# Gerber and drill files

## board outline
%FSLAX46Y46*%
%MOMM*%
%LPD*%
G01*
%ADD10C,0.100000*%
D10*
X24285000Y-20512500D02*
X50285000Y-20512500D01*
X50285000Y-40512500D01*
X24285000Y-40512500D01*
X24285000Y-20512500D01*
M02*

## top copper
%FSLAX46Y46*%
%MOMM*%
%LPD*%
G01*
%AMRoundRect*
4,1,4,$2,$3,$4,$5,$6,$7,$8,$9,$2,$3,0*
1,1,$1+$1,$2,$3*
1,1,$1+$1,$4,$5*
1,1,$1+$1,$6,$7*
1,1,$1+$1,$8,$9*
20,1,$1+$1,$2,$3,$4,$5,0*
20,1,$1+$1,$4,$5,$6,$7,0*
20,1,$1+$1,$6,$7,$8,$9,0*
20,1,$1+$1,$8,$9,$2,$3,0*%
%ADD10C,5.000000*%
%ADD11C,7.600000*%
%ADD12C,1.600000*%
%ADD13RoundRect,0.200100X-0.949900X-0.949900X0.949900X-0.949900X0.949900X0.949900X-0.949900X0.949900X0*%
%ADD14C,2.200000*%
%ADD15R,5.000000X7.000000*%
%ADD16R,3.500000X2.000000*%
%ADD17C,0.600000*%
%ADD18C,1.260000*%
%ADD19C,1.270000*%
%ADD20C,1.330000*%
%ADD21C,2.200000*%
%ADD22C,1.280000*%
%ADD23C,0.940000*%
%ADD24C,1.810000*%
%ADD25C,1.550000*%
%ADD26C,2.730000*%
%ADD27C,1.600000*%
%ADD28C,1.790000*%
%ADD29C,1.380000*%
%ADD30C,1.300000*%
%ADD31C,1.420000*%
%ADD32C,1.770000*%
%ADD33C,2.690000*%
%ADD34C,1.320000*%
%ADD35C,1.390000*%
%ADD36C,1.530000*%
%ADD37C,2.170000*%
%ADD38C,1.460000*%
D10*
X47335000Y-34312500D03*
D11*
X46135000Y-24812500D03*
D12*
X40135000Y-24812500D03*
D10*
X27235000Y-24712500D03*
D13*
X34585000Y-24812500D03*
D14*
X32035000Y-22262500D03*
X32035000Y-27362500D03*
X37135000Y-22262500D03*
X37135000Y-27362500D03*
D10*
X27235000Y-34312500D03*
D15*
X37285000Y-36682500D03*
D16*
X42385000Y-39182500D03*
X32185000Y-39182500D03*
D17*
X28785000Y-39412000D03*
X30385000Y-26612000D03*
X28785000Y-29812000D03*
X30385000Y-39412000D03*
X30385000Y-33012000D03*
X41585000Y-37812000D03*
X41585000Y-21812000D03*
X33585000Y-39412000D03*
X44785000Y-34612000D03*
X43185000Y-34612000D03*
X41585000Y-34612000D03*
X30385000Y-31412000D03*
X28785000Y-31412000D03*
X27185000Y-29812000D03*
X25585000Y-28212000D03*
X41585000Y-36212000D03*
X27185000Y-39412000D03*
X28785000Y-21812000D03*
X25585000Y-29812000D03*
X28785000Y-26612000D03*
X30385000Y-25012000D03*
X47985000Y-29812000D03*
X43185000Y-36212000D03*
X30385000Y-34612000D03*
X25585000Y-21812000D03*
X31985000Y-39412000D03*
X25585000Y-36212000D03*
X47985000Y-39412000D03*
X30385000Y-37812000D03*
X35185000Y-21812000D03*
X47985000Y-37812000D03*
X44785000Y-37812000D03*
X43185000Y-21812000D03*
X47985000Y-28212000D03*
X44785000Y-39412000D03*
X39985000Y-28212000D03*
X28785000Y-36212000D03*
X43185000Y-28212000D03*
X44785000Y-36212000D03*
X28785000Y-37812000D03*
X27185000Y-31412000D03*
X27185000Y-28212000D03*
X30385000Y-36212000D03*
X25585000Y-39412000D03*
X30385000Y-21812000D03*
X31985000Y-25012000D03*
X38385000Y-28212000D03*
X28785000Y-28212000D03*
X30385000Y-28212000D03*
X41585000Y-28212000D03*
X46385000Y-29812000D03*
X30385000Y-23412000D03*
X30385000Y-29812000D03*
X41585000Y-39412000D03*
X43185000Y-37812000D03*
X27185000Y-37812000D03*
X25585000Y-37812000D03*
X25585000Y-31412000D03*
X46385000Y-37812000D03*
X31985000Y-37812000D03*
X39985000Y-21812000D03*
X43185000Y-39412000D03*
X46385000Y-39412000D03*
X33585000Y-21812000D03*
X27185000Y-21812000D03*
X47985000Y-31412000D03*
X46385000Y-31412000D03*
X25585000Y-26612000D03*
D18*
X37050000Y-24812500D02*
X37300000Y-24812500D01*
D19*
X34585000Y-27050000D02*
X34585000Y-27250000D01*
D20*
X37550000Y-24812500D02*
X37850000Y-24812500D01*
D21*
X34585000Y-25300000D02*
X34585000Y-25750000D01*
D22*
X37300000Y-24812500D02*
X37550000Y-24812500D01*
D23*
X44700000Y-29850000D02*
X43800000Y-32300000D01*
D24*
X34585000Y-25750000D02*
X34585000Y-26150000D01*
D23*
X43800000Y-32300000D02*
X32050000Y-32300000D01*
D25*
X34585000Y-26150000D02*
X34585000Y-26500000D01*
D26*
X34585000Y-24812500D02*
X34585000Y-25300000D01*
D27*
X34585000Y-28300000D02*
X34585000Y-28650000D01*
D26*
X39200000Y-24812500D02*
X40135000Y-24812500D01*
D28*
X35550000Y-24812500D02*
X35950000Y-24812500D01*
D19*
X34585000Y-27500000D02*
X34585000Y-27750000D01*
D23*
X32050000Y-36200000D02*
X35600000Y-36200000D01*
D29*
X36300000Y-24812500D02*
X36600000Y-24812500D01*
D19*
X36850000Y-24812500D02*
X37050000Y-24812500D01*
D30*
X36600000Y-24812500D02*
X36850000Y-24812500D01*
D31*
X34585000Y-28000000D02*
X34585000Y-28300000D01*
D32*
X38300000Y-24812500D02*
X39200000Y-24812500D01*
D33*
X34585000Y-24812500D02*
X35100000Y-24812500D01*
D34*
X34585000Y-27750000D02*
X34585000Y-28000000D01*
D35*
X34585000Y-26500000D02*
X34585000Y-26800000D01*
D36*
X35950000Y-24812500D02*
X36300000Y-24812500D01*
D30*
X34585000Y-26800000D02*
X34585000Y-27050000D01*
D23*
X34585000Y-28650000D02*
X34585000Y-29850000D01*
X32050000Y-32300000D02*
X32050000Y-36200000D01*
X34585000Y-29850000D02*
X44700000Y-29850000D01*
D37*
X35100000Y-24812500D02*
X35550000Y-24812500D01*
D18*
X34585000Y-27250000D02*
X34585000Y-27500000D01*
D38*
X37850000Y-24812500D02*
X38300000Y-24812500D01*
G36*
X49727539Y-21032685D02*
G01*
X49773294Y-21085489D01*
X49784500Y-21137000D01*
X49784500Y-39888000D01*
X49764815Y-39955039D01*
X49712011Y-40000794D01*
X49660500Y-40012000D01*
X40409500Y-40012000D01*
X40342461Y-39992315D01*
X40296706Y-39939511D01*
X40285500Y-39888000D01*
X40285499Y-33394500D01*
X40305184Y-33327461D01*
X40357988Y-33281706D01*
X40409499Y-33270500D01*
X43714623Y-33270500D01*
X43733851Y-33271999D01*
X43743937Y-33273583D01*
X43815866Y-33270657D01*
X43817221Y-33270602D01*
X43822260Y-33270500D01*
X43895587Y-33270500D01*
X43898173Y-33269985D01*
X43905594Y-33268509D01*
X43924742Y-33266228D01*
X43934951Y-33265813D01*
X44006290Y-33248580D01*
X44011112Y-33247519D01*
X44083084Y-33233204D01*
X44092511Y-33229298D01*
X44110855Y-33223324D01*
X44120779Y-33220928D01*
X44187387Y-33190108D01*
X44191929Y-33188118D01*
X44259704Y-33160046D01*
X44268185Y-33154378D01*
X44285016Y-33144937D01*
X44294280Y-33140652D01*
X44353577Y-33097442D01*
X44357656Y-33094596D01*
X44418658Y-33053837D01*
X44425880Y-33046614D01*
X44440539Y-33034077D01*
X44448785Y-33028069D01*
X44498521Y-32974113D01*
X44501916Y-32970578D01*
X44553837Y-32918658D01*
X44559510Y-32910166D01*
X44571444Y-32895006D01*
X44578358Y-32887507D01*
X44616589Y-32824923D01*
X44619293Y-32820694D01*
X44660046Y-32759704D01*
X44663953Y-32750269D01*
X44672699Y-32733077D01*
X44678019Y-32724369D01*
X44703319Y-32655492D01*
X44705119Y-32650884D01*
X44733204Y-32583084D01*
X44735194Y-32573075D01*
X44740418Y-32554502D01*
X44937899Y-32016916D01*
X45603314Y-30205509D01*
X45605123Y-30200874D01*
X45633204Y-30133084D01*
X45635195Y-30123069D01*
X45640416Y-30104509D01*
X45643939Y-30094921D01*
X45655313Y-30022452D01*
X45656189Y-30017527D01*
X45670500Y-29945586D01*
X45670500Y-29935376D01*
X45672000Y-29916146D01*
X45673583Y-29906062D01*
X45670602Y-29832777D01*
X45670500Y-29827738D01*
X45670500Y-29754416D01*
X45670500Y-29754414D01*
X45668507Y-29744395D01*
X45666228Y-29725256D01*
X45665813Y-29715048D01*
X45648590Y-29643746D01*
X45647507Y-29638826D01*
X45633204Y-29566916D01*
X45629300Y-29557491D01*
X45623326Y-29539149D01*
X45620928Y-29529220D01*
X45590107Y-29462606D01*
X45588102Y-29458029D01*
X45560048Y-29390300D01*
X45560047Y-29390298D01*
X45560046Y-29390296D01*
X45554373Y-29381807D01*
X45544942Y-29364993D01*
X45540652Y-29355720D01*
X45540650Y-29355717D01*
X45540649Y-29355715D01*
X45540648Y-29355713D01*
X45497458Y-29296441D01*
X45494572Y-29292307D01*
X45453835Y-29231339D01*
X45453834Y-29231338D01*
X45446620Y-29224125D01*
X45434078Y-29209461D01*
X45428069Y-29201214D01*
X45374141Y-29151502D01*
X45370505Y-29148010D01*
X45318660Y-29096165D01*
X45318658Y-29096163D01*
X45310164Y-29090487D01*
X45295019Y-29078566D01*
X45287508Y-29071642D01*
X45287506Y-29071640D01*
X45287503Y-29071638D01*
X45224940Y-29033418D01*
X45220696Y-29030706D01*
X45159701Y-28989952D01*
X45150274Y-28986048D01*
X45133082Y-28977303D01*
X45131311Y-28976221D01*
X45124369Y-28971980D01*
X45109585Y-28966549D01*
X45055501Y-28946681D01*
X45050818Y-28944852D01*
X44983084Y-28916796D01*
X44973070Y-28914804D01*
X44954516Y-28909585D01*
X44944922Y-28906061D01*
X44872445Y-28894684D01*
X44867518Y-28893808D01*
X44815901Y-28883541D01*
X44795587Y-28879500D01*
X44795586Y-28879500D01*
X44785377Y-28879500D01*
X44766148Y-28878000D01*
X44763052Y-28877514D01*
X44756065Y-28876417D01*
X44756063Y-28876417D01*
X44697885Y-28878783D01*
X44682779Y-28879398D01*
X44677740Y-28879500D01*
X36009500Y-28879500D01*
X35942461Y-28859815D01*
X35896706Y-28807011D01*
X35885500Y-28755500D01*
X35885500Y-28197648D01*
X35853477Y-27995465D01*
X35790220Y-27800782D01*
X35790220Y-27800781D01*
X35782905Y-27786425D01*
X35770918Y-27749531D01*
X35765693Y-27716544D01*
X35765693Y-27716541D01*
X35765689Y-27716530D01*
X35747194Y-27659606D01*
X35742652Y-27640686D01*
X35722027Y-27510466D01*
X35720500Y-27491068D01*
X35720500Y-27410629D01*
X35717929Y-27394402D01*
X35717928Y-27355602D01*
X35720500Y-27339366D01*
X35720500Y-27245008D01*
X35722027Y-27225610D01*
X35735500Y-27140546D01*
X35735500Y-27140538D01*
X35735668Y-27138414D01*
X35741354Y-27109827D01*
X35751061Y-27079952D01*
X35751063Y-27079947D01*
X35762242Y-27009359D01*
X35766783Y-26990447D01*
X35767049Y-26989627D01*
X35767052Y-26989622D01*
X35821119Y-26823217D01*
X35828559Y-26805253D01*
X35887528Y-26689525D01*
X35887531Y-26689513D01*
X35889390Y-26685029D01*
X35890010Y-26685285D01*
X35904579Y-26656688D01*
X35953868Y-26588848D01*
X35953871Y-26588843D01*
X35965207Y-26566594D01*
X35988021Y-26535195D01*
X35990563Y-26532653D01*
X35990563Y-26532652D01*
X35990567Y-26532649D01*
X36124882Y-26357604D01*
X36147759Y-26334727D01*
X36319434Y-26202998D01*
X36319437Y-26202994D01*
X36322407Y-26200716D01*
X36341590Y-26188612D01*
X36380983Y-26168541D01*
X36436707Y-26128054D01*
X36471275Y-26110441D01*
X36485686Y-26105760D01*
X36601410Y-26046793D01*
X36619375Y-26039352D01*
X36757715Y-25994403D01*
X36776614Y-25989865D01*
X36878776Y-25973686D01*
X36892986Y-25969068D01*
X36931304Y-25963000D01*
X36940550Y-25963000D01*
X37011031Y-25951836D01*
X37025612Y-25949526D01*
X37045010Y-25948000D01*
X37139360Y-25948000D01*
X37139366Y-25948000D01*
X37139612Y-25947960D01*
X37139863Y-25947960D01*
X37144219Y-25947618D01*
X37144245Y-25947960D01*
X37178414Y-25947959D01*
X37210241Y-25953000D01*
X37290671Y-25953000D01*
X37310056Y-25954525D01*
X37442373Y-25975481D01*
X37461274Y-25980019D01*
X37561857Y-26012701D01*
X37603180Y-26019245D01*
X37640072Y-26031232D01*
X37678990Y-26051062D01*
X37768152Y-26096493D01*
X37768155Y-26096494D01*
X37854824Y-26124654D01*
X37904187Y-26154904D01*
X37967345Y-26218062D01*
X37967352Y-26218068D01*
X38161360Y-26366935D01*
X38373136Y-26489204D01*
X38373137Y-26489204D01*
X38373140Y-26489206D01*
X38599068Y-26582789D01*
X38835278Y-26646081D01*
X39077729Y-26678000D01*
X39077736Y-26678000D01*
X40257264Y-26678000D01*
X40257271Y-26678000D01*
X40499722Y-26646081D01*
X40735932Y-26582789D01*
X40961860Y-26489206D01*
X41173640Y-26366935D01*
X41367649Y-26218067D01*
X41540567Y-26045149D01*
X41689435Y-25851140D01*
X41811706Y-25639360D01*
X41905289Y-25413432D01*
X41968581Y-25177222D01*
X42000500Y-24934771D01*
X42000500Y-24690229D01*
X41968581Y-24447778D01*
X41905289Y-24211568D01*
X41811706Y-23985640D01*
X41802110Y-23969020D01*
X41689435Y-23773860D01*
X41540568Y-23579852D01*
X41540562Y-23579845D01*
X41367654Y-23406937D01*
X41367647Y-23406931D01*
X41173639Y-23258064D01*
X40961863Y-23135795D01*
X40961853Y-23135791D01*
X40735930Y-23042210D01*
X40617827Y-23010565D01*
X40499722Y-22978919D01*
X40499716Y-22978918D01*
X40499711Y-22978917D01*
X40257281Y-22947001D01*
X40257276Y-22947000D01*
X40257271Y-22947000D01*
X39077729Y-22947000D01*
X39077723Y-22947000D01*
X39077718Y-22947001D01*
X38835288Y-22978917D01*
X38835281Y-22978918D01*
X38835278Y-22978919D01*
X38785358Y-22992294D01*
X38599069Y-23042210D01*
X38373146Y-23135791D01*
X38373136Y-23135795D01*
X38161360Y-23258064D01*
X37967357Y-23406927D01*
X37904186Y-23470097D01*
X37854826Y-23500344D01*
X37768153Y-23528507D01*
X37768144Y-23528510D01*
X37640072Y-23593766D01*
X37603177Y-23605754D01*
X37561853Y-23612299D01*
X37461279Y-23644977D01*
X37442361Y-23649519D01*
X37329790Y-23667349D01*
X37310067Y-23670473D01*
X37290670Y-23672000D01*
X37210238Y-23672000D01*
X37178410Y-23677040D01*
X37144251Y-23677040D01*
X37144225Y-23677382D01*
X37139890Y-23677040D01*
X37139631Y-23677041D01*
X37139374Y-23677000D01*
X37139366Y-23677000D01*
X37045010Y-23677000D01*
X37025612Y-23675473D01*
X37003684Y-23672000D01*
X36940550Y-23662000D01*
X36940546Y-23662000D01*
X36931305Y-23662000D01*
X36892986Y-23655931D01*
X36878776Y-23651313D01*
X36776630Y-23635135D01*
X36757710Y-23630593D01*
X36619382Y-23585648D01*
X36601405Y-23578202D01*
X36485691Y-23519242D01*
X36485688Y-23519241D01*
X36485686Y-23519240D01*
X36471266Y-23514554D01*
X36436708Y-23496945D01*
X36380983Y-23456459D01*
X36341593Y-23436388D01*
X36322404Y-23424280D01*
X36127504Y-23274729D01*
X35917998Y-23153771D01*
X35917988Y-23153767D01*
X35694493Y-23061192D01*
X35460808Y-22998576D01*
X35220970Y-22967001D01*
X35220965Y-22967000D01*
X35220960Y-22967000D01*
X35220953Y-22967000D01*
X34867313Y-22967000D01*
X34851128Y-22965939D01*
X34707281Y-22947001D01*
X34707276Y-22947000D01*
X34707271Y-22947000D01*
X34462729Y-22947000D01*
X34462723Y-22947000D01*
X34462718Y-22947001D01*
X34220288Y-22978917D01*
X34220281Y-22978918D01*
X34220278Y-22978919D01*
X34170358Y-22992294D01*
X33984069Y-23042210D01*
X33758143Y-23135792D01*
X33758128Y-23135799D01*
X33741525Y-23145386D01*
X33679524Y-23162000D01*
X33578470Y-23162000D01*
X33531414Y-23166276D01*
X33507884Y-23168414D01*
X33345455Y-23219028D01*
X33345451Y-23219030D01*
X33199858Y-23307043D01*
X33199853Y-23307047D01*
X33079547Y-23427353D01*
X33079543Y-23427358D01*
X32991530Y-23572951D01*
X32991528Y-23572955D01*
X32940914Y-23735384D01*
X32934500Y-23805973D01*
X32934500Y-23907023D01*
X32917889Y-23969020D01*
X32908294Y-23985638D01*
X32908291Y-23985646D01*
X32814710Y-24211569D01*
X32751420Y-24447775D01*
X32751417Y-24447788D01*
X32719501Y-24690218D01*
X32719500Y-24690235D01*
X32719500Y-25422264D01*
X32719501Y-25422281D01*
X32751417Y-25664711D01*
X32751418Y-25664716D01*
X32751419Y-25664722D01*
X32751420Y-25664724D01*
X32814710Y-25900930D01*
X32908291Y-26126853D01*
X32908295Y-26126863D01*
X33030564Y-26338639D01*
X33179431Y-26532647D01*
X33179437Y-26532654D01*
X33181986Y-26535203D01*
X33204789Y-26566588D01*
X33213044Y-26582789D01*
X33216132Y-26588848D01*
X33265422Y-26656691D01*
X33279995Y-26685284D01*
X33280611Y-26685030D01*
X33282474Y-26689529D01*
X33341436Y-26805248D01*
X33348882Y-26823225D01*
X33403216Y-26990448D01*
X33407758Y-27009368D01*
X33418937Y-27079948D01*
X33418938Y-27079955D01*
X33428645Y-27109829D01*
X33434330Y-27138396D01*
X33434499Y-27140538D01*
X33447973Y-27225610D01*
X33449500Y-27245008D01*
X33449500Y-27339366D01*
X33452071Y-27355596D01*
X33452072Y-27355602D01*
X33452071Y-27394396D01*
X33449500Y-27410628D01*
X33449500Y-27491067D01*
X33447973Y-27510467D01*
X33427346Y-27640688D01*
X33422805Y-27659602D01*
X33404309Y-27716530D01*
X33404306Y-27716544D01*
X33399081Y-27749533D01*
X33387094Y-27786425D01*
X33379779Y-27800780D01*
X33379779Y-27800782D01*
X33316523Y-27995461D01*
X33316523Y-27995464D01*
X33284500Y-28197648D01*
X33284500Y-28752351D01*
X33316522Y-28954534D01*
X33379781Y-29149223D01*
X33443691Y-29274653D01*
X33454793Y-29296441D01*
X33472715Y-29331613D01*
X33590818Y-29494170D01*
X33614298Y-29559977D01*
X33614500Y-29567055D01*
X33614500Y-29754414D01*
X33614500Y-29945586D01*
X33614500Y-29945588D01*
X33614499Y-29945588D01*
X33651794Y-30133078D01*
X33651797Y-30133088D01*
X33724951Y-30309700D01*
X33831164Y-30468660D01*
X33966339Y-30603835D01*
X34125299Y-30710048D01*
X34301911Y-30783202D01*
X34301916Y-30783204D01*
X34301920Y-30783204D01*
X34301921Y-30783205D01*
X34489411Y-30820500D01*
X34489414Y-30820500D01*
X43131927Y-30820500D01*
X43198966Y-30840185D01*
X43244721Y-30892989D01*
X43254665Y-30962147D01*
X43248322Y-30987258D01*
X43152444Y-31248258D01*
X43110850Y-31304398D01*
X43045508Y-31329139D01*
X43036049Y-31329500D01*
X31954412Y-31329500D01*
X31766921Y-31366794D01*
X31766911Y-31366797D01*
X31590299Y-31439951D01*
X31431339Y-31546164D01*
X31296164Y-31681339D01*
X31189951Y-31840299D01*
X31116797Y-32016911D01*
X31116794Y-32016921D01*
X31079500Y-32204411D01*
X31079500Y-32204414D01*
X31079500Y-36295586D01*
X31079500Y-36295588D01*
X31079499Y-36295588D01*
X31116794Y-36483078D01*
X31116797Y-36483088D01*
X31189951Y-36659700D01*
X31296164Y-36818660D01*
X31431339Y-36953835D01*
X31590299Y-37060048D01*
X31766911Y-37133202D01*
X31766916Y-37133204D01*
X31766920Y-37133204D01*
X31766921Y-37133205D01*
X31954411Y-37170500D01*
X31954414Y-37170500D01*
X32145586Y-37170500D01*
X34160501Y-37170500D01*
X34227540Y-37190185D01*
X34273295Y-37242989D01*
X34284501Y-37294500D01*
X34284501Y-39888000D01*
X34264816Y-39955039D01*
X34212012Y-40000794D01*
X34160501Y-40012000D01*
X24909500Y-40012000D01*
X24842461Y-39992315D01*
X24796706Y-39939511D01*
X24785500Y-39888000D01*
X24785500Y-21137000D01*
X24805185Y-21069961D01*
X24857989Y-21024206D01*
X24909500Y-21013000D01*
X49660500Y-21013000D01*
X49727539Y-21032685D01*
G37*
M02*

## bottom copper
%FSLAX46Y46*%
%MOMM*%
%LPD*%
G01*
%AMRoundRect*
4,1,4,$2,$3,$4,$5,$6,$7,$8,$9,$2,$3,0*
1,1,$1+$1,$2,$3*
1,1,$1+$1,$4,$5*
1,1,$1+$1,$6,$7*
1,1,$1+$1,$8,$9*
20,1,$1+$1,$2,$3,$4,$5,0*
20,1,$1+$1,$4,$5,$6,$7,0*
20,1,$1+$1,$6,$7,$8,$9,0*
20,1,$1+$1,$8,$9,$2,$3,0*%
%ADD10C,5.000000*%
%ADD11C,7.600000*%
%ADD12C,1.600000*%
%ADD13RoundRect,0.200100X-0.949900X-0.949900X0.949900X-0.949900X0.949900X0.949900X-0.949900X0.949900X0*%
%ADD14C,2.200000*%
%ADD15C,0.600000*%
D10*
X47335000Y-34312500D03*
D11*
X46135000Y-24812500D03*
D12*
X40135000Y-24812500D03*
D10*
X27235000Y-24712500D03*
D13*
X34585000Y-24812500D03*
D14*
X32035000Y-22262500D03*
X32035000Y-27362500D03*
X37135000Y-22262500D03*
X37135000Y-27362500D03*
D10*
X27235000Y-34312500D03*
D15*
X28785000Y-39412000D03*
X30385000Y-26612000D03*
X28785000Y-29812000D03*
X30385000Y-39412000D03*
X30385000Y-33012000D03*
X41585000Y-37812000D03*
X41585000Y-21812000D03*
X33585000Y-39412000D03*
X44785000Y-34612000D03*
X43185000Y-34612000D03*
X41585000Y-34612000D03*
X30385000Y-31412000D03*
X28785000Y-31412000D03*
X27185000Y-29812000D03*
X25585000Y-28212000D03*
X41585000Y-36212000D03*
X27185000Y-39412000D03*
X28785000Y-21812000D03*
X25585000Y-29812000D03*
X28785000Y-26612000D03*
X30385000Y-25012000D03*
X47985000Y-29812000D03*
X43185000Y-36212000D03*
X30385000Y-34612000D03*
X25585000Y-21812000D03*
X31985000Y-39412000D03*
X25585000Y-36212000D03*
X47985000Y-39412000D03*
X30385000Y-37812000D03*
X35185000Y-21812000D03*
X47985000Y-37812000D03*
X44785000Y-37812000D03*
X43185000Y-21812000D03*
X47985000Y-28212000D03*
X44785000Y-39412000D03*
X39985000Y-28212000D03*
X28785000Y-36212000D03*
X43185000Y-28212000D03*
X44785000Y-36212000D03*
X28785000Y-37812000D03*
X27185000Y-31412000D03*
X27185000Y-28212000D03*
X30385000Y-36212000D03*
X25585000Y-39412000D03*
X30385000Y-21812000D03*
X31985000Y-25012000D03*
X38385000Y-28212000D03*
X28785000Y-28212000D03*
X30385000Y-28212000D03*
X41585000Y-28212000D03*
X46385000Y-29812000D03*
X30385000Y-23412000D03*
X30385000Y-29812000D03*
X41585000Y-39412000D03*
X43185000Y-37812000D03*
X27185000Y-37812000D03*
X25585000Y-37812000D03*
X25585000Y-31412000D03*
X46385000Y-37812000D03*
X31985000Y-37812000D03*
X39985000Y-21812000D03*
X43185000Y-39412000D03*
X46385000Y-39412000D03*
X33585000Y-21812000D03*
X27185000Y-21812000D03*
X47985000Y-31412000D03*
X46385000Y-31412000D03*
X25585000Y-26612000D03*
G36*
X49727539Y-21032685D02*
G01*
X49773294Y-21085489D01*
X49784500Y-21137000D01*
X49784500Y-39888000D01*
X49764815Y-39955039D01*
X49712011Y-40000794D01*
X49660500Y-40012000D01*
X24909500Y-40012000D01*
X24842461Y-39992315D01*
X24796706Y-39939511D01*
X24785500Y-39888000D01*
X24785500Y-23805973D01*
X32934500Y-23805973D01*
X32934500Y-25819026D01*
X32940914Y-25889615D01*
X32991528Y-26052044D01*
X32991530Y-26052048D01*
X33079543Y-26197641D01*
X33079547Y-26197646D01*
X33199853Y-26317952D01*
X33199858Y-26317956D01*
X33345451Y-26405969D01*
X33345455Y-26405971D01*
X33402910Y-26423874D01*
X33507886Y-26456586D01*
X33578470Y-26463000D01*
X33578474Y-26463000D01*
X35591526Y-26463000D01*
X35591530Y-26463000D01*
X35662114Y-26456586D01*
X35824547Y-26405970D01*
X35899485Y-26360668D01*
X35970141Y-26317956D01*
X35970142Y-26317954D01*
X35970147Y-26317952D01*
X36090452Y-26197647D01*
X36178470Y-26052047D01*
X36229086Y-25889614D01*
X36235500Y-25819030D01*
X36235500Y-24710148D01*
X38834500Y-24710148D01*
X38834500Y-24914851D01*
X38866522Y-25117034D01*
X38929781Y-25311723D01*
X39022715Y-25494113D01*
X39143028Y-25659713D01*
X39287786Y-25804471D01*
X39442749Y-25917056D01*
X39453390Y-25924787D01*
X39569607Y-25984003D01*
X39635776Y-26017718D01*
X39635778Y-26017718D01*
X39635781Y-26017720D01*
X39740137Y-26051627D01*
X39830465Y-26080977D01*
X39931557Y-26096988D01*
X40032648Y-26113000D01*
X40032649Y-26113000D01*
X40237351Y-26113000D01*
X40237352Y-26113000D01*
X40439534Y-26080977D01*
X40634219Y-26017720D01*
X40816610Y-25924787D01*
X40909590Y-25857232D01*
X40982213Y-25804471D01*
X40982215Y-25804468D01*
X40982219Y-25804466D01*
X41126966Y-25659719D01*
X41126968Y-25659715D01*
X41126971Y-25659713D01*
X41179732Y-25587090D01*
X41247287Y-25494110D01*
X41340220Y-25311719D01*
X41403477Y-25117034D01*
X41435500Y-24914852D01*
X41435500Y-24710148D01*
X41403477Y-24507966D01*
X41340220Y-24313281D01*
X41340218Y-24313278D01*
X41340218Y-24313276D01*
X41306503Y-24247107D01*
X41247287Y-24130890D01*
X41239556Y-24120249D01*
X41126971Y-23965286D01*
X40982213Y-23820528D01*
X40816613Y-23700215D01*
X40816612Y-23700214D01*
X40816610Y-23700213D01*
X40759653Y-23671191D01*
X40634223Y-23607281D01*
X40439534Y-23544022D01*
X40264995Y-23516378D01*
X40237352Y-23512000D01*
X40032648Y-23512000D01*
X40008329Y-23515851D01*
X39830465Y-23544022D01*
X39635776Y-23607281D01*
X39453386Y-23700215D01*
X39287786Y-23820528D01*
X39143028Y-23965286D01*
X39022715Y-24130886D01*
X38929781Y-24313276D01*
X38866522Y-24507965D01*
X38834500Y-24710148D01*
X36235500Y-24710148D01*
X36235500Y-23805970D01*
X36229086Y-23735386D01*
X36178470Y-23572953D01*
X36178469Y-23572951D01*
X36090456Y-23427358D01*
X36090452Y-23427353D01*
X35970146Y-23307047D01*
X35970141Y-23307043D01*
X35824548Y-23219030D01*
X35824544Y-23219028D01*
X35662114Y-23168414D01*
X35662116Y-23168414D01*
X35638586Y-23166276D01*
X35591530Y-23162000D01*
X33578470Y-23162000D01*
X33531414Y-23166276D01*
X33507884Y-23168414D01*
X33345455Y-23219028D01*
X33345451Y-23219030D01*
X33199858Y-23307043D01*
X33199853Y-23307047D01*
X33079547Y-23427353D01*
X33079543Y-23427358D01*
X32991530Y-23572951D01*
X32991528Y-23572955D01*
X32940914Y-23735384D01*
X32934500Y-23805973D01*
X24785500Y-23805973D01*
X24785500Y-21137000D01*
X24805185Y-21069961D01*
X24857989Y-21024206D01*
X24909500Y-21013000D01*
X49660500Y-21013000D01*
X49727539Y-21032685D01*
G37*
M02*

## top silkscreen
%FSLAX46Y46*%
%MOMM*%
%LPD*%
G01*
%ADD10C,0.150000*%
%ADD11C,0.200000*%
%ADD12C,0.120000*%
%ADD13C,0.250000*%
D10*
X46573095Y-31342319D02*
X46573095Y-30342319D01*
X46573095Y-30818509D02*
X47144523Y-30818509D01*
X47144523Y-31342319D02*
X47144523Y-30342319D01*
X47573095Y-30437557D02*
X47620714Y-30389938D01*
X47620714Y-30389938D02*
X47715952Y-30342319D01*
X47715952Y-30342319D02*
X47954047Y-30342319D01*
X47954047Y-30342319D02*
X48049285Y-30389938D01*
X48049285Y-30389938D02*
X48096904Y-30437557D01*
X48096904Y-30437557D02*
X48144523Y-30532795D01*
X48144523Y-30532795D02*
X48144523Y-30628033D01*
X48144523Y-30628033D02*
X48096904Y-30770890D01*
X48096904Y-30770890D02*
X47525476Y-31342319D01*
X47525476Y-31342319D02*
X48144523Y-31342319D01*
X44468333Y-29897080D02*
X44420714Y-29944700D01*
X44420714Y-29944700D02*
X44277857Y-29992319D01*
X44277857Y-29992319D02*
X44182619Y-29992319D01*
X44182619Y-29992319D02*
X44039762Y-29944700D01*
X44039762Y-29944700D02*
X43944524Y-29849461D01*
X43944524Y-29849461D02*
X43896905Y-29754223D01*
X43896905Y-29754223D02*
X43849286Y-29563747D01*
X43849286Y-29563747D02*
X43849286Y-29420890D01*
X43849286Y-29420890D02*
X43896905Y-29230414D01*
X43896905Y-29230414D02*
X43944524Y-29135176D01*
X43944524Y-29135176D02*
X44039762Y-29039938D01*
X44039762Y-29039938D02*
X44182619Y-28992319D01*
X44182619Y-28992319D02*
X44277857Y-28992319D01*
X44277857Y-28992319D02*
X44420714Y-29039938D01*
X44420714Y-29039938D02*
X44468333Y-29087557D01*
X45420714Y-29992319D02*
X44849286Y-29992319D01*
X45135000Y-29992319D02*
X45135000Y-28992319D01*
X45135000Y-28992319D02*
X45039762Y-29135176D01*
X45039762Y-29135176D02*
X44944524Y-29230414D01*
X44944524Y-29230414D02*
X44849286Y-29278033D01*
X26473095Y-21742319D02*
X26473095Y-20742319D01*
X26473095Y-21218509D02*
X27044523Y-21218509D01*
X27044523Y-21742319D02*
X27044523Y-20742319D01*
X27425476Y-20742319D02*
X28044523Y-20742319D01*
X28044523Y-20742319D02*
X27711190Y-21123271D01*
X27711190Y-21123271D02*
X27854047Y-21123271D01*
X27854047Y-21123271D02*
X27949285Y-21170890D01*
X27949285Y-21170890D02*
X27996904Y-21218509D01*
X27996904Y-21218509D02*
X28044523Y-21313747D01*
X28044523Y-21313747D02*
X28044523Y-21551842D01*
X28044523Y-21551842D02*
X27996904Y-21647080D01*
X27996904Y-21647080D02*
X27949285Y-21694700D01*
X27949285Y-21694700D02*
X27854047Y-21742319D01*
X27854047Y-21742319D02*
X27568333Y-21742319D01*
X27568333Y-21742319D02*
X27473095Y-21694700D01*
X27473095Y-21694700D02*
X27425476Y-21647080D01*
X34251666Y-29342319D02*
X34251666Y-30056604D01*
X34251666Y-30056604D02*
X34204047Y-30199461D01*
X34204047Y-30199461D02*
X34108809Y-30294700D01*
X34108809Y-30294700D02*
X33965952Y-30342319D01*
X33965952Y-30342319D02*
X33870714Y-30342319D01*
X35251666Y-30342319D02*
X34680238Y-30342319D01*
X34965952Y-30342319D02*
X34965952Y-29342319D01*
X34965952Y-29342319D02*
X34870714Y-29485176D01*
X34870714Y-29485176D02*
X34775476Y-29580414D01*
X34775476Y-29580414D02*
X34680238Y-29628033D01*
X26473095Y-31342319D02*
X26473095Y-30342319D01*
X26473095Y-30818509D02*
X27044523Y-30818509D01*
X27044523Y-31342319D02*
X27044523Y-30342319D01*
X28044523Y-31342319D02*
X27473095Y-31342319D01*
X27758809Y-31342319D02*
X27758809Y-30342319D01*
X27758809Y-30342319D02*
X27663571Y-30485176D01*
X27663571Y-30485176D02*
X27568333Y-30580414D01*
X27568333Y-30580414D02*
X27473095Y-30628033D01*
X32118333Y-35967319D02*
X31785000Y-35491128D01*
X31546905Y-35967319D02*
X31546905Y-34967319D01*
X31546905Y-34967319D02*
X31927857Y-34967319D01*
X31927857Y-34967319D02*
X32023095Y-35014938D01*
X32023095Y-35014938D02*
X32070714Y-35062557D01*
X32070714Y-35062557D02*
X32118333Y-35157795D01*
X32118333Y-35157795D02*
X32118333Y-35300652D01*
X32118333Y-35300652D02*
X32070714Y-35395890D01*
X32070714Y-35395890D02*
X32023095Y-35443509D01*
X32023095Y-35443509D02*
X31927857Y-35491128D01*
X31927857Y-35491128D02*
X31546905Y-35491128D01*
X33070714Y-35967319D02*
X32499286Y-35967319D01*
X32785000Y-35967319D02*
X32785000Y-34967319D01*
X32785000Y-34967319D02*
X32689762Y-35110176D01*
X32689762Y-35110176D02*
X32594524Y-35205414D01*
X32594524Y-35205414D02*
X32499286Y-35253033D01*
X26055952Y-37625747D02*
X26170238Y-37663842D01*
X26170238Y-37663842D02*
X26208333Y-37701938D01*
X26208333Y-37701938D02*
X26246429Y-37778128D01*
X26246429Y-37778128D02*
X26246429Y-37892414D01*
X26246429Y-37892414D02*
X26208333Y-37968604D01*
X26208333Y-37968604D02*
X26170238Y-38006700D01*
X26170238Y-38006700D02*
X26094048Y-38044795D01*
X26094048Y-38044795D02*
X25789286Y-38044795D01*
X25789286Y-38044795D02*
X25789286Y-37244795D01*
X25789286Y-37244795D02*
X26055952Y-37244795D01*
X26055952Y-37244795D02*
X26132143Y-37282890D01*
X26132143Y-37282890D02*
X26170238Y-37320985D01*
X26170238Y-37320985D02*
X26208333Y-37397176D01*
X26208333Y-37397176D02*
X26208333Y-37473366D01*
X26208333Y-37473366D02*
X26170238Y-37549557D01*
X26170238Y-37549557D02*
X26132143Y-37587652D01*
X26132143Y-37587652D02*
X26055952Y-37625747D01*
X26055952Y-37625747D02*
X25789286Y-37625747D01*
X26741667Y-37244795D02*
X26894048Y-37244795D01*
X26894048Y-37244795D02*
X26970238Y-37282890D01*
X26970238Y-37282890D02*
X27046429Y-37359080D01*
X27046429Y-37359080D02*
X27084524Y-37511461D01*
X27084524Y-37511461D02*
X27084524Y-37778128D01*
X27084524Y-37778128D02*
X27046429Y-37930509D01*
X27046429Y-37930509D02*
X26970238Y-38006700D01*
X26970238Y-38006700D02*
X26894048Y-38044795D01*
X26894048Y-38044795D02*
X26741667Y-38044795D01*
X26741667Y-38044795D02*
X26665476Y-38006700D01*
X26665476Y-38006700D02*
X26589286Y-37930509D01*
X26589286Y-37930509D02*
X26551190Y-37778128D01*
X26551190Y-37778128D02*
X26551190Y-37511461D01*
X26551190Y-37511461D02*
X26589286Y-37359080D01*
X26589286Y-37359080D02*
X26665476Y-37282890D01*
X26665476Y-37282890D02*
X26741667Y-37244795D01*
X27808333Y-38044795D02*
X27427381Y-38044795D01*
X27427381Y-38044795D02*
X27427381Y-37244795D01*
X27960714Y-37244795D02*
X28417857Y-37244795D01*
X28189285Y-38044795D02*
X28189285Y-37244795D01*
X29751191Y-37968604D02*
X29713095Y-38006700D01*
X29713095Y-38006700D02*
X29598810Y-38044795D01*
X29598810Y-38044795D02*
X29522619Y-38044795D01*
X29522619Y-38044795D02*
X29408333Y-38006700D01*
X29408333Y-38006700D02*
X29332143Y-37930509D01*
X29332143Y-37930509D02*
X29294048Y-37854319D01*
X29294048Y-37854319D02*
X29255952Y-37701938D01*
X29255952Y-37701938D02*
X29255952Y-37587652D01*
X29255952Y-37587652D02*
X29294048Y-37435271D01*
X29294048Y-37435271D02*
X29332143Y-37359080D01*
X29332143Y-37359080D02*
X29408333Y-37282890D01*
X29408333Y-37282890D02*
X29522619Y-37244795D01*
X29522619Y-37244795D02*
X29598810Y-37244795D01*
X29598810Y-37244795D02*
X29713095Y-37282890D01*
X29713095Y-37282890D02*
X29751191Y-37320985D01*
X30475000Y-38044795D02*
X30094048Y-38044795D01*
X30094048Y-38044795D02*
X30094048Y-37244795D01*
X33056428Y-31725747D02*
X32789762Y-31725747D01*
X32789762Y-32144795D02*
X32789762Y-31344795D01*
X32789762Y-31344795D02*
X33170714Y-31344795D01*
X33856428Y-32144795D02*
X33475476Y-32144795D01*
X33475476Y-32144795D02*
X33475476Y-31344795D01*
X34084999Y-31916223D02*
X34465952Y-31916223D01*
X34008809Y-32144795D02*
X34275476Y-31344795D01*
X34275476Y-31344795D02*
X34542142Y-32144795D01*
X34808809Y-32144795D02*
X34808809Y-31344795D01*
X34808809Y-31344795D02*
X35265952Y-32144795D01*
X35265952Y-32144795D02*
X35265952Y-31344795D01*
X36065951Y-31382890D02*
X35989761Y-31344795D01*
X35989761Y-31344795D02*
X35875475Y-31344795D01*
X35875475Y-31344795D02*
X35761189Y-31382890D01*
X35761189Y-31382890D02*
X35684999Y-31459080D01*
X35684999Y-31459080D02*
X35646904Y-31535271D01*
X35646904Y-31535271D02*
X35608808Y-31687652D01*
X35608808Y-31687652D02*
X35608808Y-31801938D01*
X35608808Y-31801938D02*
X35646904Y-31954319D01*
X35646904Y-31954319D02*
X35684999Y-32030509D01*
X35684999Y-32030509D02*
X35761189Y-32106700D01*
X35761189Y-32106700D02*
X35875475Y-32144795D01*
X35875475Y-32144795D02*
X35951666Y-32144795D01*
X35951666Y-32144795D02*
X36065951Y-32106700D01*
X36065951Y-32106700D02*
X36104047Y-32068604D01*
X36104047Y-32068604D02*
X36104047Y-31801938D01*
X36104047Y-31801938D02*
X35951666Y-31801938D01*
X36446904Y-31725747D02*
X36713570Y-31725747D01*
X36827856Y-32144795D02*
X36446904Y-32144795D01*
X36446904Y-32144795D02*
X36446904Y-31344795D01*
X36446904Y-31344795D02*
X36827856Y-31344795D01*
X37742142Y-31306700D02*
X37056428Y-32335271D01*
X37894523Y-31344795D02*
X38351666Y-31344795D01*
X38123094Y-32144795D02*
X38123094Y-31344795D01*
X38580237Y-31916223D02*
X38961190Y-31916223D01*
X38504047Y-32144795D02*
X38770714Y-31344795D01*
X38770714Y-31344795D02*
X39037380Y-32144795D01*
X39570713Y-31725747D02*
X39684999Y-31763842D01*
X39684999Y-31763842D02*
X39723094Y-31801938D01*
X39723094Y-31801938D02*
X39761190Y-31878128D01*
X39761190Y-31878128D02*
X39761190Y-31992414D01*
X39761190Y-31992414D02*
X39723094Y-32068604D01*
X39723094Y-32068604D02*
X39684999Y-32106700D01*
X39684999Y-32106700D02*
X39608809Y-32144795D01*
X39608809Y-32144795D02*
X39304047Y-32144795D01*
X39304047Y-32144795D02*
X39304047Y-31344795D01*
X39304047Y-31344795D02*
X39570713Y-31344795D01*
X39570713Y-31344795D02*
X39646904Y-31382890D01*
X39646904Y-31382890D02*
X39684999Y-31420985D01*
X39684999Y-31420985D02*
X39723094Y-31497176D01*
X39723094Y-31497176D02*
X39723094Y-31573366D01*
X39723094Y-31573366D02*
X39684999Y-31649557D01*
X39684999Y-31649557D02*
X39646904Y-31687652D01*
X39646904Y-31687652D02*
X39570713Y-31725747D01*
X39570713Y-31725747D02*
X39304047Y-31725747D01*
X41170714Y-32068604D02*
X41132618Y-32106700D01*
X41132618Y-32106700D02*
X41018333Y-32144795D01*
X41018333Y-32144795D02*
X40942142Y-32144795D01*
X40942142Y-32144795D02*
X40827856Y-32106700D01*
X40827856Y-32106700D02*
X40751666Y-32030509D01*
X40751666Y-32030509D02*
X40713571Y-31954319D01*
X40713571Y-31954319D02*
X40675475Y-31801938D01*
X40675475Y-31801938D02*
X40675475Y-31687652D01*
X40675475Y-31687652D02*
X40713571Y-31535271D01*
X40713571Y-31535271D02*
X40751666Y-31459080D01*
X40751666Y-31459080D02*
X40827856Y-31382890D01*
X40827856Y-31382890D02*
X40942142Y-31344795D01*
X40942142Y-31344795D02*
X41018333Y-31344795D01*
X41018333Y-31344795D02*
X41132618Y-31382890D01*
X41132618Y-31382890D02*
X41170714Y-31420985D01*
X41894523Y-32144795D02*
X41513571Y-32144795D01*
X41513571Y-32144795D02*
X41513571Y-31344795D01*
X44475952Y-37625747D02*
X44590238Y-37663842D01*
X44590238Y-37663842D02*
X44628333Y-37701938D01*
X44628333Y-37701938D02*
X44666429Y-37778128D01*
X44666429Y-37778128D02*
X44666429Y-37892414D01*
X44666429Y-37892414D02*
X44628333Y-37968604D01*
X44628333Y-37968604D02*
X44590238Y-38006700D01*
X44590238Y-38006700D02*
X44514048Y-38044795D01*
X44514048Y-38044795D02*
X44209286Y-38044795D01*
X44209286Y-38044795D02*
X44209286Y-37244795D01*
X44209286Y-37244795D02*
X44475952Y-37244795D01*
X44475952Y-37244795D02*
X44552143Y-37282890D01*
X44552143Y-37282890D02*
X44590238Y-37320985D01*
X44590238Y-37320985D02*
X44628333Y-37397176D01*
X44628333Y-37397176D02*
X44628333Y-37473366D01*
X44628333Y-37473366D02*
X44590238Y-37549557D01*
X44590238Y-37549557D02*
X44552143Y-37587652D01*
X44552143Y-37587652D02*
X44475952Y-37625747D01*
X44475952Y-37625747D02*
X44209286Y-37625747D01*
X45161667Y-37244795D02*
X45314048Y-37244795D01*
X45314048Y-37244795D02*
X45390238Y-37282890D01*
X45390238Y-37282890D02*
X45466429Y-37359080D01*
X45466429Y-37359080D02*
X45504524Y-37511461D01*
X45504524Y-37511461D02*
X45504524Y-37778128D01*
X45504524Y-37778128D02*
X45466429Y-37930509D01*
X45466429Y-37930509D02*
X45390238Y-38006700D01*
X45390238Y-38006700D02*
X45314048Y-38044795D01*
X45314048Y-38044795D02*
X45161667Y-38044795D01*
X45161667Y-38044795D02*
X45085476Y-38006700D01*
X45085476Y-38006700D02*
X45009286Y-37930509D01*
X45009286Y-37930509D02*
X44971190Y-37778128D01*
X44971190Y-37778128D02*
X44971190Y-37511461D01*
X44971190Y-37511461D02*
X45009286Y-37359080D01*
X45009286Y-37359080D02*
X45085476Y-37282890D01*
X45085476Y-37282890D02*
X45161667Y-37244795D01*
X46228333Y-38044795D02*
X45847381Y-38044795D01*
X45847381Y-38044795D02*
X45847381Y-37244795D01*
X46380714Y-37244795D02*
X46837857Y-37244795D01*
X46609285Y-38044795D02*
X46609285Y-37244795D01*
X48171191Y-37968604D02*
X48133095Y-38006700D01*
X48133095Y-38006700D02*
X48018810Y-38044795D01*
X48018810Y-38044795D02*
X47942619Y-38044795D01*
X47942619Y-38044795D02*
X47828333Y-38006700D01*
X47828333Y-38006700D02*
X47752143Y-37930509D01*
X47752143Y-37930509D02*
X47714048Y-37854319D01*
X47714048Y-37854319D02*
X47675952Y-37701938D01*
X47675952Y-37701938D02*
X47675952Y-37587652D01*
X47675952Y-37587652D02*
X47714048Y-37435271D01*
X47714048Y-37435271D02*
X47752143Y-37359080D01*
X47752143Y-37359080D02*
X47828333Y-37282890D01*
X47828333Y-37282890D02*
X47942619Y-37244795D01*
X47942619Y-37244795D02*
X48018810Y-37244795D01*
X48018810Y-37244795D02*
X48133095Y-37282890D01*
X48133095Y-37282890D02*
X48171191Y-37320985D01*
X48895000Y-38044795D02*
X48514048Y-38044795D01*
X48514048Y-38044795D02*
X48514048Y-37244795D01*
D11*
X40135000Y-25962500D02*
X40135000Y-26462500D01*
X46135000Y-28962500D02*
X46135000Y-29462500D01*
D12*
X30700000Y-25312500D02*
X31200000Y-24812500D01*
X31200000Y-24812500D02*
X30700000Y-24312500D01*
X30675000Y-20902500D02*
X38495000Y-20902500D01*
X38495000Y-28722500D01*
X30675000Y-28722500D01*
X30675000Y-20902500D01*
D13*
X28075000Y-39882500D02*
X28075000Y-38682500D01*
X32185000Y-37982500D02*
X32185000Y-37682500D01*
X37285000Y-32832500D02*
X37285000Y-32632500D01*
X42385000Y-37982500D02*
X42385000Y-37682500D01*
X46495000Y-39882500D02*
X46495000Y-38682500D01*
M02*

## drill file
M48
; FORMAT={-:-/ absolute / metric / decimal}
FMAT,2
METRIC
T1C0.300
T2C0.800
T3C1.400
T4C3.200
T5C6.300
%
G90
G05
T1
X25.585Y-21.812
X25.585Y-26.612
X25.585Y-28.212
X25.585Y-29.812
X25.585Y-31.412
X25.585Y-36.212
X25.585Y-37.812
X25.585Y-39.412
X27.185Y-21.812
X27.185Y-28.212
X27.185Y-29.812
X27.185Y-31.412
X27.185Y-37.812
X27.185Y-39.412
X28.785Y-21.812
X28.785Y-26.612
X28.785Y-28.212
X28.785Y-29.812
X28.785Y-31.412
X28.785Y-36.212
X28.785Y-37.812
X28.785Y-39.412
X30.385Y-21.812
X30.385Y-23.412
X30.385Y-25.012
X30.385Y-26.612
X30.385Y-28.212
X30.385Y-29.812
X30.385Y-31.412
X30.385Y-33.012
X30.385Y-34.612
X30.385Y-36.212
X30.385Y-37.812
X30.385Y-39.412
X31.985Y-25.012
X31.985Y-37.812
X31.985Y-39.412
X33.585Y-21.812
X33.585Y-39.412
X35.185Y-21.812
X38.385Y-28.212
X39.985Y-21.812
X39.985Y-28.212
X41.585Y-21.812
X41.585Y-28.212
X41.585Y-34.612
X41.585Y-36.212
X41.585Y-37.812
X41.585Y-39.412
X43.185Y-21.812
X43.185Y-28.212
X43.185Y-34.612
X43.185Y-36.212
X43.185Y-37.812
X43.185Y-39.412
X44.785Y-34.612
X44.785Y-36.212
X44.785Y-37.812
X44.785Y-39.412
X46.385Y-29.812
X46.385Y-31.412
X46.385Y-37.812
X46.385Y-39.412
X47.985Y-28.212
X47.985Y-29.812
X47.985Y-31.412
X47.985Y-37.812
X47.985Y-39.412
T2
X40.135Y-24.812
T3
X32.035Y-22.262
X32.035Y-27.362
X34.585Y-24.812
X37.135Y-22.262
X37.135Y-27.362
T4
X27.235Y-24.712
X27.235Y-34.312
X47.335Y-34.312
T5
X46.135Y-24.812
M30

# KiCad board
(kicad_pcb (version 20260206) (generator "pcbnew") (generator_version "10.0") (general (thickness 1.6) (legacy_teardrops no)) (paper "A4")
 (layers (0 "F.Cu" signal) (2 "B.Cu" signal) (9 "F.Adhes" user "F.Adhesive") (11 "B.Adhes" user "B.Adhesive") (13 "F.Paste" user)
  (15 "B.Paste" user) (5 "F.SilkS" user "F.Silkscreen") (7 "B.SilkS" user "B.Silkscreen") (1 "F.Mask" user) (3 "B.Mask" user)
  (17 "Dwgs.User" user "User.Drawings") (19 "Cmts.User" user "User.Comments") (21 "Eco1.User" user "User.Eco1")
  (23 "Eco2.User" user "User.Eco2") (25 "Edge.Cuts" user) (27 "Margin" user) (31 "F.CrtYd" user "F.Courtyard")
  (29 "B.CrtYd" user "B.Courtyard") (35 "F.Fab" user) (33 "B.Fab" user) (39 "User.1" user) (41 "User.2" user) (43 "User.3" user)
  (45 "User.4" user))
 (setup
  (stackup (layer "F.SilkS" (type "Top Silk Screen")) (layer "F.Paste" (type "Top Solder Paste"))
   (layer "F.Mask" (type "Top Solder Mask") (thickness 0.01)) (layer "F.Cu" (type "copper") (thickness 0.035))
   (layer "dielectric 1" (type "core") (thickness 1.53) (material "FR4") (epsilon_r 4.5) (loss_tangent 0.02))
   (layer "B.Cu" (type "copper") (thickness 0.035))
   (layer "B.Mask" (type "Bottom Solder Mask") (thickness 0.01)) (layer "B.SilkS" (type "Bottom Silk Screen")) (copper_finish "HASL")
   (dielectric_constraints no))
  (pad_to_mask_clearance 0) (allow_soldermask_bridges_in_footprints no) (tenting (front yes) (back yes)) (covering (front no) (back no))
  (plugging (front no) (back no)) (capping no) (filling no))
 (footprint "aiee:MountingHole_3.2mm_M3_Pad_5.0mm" (layer "F.Cu") (at 47.335 34.3125)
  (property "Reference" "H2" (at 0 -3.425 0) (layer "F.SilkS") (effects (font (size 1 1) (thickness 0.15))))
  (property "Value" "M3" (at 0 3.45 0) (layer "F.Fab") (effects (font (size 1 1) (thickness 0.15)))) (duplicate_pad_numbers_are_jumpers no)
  (pad "1" thru_hole circle (at 0 0) (size 5 5) (drill 3.2) (layers "*.Cu" "*.Mask") (remove_unused_layers no) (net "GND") (zone_connect 2)))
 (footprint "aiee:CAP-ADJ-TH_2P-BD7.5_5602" (layer "F.Cu") (at 46.135 24.8125 180)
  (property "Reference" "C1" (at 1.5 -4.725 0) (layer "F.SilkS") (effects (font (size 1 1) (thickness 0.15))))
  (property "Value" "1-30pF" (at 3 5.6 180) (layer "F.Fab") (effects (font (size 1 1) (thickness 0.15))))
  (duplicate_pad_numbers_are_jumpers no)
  (fp_line (start 6 -1.15) (end 6 -1.65) (stroke (width 0.2) (type solid)) (layer "F.SilkS"))
  (fp_line (start 0 -4.15) (end 0 -4.65) (stroke (width 0.2) (type solid)) (layer "F.SilkS"))
  (pad "1" thru_hole circle (at 0 0 180) (size 7.6 7.6) (drill 6.3) (layers "*.Cu" "*.Mask") (remove_unused_layers no) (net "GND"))
  (pad "2" thru_hole circle (at 6 0 180) (size 1.6 1.6) (drill 0.8) (layers "*.Cu" "*.Mask") (remove_unused_layers no) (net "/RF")))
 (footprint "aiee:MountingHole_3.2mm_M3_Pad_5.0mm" (layer "F.Cu") (at 27.235 24.7125)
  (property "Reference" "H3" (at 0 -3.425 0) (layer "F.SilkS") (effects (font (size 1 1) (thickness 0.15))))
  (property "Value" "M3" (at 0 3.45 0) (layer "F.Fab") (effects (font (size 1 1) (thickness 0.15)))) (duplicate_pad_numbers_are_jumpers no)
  (pad "1" thru_hole circle (at 0 0) (size 5 5) (drill 3.2) (layers "*.Cu" "*.Mask") (remove_unused_layers no) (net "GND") (zone_connect 2)))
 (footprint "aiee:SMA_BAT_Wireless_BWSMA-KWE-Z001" (layer "F.Cu") (at 34.585 24.8125)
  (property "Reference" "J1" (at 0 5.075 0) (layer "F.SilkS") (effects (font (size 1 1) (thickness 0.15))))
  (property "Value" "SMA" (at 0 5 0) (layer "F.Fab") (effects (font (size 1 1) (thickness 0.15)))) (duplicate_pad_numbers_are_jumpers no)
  (fp_line (start -3.885 0.5) (end -3.385 0) (stroke (width 0.12) (type solid)) (layer "F.SilkS"))
  (fp_line (start -3.385 0) (end -3.885 -0.5) (stroke (width 0.12) (type solid)) (layer "F.SilkS"))
  (fp_rect (start -3.91 -3.91) (end 3.91 3.91) (stroke (width 0.12) (type default)) (fill no) (layer "F.SilkS"))
  (pad "1" thru_hole roundrect (at 0 0) (size 2.3 2.3) (drill 1.4) (layers "*.Cu" "*.Mask") (remove_unused_layers yes) (keep_end_layers yes)
   (zone_layer_connections) (roundrect_rratio 0.087) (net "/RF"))
  (pad "2" thru_hole circle (at -2.55 -2.55) (size 2.2 2.2) (drill 1.4) (layers "*.Cu" "*.Mask") (remove_unused_layers yes)
   (keep_end_layers yes) (zone_layer_connections) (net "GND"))
  (pad "2" thru_hole circle (at -2.55 2.55) (size 2.2 2.2) (drill 1.4) (layers "*.Cu" "*.Mask") (remove_unused_layers yes)
   (keep_end_layers yes) (zone_layer_connections) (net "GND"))
  (pad "2" thru_hole circle (at 2.55 -2.55) (size 2.2 2.2) (drill 1.4) (layers "*.Cu" "*.Mask") (remove_unused_layers yes)
   (keep_end_layers yes) (zone_layer_connections) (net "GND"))
  (pad "2" thru_hole circle (at 2.55 2.55) (size 2.2 2.2) (drill 1.4) (layers "*.Cu" "*.Mask") (remove_unused_layers yes)
   (keep_end_layers yes) (zone_layer_connections) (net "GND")))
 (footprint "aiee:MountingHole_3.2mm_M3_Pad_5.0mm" (layer "F.Cu") (at 27.235 34.3125)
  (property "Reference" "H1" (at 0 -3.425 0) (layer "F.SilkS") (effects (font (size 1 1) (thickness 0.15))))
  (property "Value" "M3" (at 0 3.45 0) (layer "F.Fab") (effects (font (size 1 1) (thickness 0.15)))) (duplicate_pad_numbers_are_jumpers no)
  (pad "1" thru_hole circle (at 0 0) (size 5 5) (drill 3.2) (layers "*.Cu" "*.Mask") (remove_unused_layers no) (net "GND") (zone_connect 2)))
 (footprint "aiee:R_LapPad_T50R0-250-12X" (layer "F.Cu") (at 37.285 40.1825 180)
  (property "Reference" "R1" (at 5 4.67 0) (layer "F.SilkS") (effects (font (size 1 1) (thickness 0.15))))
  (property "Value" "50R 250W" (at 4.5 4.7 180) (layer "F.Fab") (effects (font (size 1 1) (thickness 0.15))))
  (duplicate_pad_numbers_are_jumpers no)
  (fp_line (start 9.21 0.3) (end 9.21 1.5) (stroke (width 0.25) (type solid)) (layer "F.SilkS"))
  (fp_line (start 5.1 2.2) (end 5.1 2.5) (stroke (width 0.25) (type solid)) (layer "F.SilkS"))
  (fp_line (start 0 7.35) (end 0 7.55) (stroke (width 0.25) (type solid)) (layer "F.SilkS"))
  (fp_line (start -5.1 2.2) (end -5.1 2.5) (stroke (width 0.25) (type solid)) (layer "F.SilkS"))
  (fp_line (start -9.21 0.3) (end -9.21 1.5) (stroke (width 0.25) (type solid)) (layer "F.SilkS"))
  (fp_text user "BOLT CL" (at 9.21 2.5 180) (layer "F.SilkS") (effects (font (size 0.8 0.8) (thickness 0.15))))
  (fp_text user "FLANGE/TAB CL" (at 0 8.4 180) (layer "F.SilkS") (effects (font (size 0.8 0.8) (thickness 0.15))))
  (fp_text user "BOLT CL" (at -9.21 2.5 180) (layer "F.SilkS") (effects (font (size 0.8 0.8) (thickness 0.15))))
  (pad "1" smd rect (at 0 3.5 180) (size 5 7) (layers "F.Cu" "F.Mask" "F.Paste") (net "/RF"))
  (pad "2" smd rect (at -5.1 1 180) (size 3.5 2) (layers "F.Cu" "F.Mask" "F.Paste") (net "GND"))
  (pad "2" smd rect (at 5.1 1 180) (size 3.5 2) (layers "F.Cu" "F.Mask" "F.Paste") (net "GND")))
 (gr_rect (start 24.285 20.5125) (end 50.285 40.5125) (stroke (width 0.1) (type default)) (fill no) (layer "Edge.Cuts"))
 (via (at 28.785 39.412) (size 0.6) (drill 0.3) (layers "F.Cu" "B.Cu") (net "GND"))
 (via (at 30.385 26.612) (size 0.6) (drill 0.3) (layers "F.Cu" "B.Cu") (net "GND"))
 (via (at 28.785 29.812) (size 0.6) (drill 0.3) (layers "F.Cu" "B.Cu") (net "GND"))
 (via (at 30.385 39.412) (size 0.6) (drill 0.3) (layers "F.Cu" "B.Cu") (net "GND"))
 (via (at 30.385 33.012) (size 0.6) (drill 0.3) (layers "F.Cu" "B.Cu") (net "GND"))
 (via (at 41.585 37.812) (size 0.6) (drill 0.3) (layers "F.Cu" "B.Cu") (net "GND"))
 (via (at 41.585 21.812) (size 0.6) (drill 0.3) (layers "F.Cu" "B.Cu") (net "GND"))
 (via (at 33.585 39.412) (size 0.6) (drill 0.3) (layers "F.Cu" "B.Cu") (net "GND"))
 (via (at 44.785 34.612) (size 0.6) (drill 0.3) (layers "F.Cu" "B.Cu") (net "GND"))
 (via (at 43.185 34.612) (size 0.6) (drill 0.3) (layers "F.Cu" "B.Cu") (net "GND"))
 (via (at 41.585 34.612) (size 0.6) (drill 0.3) (layers "F.Cu" "B.Cu") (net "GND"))
 (via (at 30.385 31.412) (size 0.6) (drill 0.3) (layers "F.Cu" "B.Cu") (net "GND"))
 (via (at 28.785 31.412) (size 0.6) (drill 0.3) (layers "F.Cu" "B.Cu") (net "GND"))
 (via (at 27.185 29.812) (size 0.6) (drill 0.3) (layers "F.Cu" "B.Cu") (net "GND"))
 (via (at 25.585 28.212) (size 0.6) (drill 0.3) (layers "F.Cu" "B.Cu") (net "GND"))
 (via (at 41.585 36.212) (size 0.6) (drill 0.3) (layers "F.Cu" "B.Cu") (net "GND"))
 (via (at 27.185 39.412) (size 0.6) (drill 0.3) (layers "F.Cu" "B.Cu") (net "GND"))
 (via (at 28.785 21.812) (size 0.6) (drill 0.3) (layers "F.Cu" "B.Cu") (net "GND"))
 (via (at 25.585 29.812) (size 0.6) (drill 0.3) (layers "F.Cu" "B.Cu") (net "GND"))
 (via (at 28.785 26.612) (size 0.6) (drill 0.3) (layers "F.Cu" "B.Cu") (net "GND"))
 (via (at 30.385 25.012) (size 0.6) (drill 0.3) (layers "F.Cu" "B.Cu") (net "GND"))
 (via (at 47.985 29.812) (size 0.6) (drill 0.3) (layers "F.Cu" "B.Cu") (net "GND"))
 (via (at 43.185 36.212) (size 0.6) (drill 0.3) (layers "F.Cu" "B.Cu") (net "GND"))
 (via (at 30.385 34.612) (size 0.6) (drill 0.3) (layers "F.Cu" "B.Cu") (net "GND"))
 (via (at 25.585 21.812) (size 0.6) (drill 0.3) (layers "F.Cu" "B.Cu") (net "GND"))
 (via (at 31.985 39.412) (size 0.6) (drill 0.3) (layers "F.Cu" "B.Cu") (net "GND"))
 (via (at 25.585 36.212) (size 0.6) (drill 0.3) (layers "F.Cu" "B.Cu") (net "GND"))
 (via (at 47.985 39.412) (size 0.6) (drill 0.3) (layers "F.Cu" "B.Cu") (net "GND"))
 (via (at 30.385 37.812) (size 0.6) (drill 0.3) (layers "F.Cu" "B.Cu") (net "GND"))
 (via (at 35.185 21.812) (size 0.6) (drill 0.3) (layers "F.Cu" "B.Cu") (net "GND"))
 (via (at 47.985 37.812) (size 0.6) (drill 0.3) (layers "F.Cu" "B.Cu") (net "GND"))
 (via (at 44.785 37.812) (size 0.6) (drill 0.3) (layers "F.Cu" "B.Cu") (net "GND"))
 (via (at 43.185 21.812) (size 0.6) (drill 0.3) (layers "F.Cu" "B.Cu") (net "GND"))
 (via (at 47.985 28.212) (size 0.6) (drill 0.3) (layers "F.Cu" "B.Cu") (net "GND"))
 (via (at 44.785 39.412) (size 0.6) (drill 0.3) (layers "F.Cu" "B.Cu") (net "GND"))
 (via (at 39.985 28.212) (size 0.6) (drill 0.3) (layers "F.Cu" "B.Cu") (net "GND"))
 (via (at 28.785 36.212) (size 0.6) (drill 0.3) (layers "F.Cu" "B.Cu") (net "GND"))
 (via (at 43.185 28.212) (size 0.6) (drill 0.3) (layers "F.Cu" "B.Cu") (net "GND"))
 (via (at 44.785 36.212) (size 0.6) (drill 0.3) (layers "F.Cu" "B.Cu") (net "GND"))
 (via (at 28.785 37.812) (size 0.6) (drill 0.3) (layers "F.Cu" "B.Cu") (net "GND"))
 (via (at 27.185 31.412) (size 0.6) (drill 0.3) (layers "F.Cu" "B.Cu") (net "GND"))
 (via (at 27.185 28.212) (size 0.6) (drill 0.3) (layers "F.Cu" "B.Cu") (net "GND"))
 (via (at 30.385 36.212) (size 0.6) (drill 0.3) (layers "F.Cu" "B.Cu") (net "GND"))
 (via (at 25.585 39.412) (size 0.6) (drill 0.3) (layers "F.Cu" "B.Cu") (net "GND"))
 (via (at 30.385 21.812) (size 0.6) (drill 0.3) (layers "F.Cu" "B.Cu") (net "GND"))
 (via (at 31.985 25.012) (size 0.6) (drill 0.3) (layers "F.Cu" "B.Cu") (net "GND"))
 (via (at 38.385 28.212) (size 0.6) (drill 0.3) (layers "F.Cu" "B.Cu") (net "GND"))
 (via (at 28.785 28.212) (size 0.6) (drill 0.3) (layers "F.Cu" "B.Cu") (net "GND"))
 (via (at 30.385 28.212) (size 0.6) (drill 0.3) (layers "F.Cu" "B.Cu") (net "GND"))
 (via (at 41.585 28.212) (size 0.6) (drill 0.3) (layers "F.Cu" "B.Cu") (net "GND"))
 (via (at 46.385 29.812) (size 0.6) (drill 0.3) (layers "F.Cu" "B.Cu") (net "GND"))
 (via (at 30.385 23.412) (size 0.6) (drill 0.3) (layers "F.Cu" "B.Cu") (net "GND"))
 (via (at 30.385 29.812) (size 0.6) (drill 0.3) (layers "F.Cu" "B.Cu") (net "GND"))
 (via (at 41.585 39.412) (size 0.6) (drill 0.3) (layers "F.Cu" "B.Cu") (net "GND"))
 (via (at 43.185 37.812) (size 0.6) (drill 0.3) (layers "F.Cu" "B.Cu") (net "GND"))
 (via (at 27.185 37.812) (size 0.6) (drill 0.3) (layers "F.Cu" "B.Cu") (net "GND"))
 (via (at 25.585 37.812) (size 0.6) (drill 0.3) (layers "F.Cu" "B.Cu") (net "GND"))
 (via (at 25.585 31.412) (size 0.6) (drill 0.3) (layers "F.Cu" "B.Cu") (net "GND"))
 (via (at 46.385 37.812) (size 0.6) (drill 0.3) (layers "F.Cu" "B.Cu") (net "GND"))
 (via (at 31.985 37.812) (size 0.6) (drill 0.3) (layers "F.Cu" "B.Cu") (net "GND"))
 (via (at 39.985 21.812) (size 0.6) (drill 0.3) (layers "F.Cu" "B.Cu") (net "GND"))
 (via (at 43.185 39.412) (size 0.6) (drill 0.3) (layers "F.Cu" "B.Cu") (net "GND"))
 (via (at 46.385 39.412) (size 0.6) (drill 0.3) (layers "F.Cu" "B.Cu") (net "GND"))
 (via (at 33.585 21.812) (size 0.6) (drill 0.3) (layers "F.Cu" "B.Cu") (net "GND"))
 (via (at 27.185 21.812) (size 0.6) (drill 0.3) (layers "F.Cu" "B.Cu") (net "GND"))
 (via (at 47.985 31.412) (size 0.6) (drill 0.3) (layers "F.Cu" "B.Cu") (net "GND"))
 (via (at 46.385 31.412) (size 0.6) (drill 0.3) (layers "F.Cu" "B.Cu") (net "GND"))
 (via (at 25.585 26.612) (size 0.6) (drill 0.3) (layers "F.Cu" "B.Cu") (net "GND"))
 (segment (start 37.05 24.8125) (end 37.3 24.8125) (width 1.26) (layer "F.Cu") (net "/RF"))
 (segment (start 34.585 27.05) (end 34.585 27.25) (width 1.27) (layer "F.Cu") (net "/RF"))
 (segment (start 37.55 24.8125) (end 37.85 24.8125) (width 1.33) (layer "F.Cu") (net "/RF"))
 (segment (start 34.585 25.3) (end 34.585 25.75) (width 2.2) (layer "F.Cu") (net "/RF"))
 (segment (start 37.3 24.8125) (end 37.55 24.8125) (width 1.28) (layer "F.Cu") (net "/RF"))
 (segment (start 44.7 29.85) (end 43.8 32.3) (width 0.94) (layer "F.Cu") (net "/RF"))
 (segment (start 34.585 25.75) (end 34.585 26.15) (width 1.81) (layer "F.Cu") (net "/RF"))
 (segment (start 43.8 32.3) (end 32.05 32.3) (width 0.94) (layer "F.Cu") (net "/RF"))
 (segment (start 34.585 26.15) (end 34.585 26.5) (width 1.55) (layer "F.Cu") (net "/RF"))
 (segment (start 34.585 24.8125) (end 34.585 25.3) (width 2.73) (layer "F.Cu") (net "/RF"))
 (segment (start 34.585 28.3) (end 34.585 28.65) (width 1.6) (layer "F.Cu") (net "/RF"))
 (segment (start 39.2 24.8125) (end 40.135 24.8125) (width 2.73) (layer "F.Cu") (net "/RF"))
 (segment (start 35.55 24.8125) (end 35.95 24.8125) (width 1.79) (layer "F.Cu") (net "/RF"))
 (segment (start 34.585 27.5) (end 34.585 27.75) (width 1.27) (layer "F.Cu") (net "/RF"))
 (segment (start 32.05 36.2) (end 35.6 36.2) (width 0.94) (layer "F.Cu") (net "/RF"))
 (segment (start 36.3 24.8125) (end 36.6 24.8125) (width 1.38) (layer "F.Cu") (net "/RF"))
 (segment (start 36.85 24.8125) (end 37.05 24.8125) (width 1.27) (layer "F.Cu") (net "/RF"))
 (segment (start 36.6 24.8125) (end 36.85 24.8125) (width 1.3) (layer "F.Cu") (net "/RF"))
 (segment (start 34.585 28) (end 34.585 28.3) (width 1.42) (layer "F.Cu") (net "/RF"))
 (segment (start 38.3 24.8125) (end 39.2 24.8125) (width 1.77) (layer "F.Cu") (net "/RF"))
 (segment (start 34.585 24.8125) (end 35.1 24.8125) (width 2.69) (layer "F.Cu") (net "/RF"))
 (segment (start 34.585 27.75) (end 34.585 28) (width 1.32) (layer "F.Cu") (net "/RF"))
 (segment (start 34.585 26.5) (end 34.585 26.8) (width 1.39) (layer "F.Cu") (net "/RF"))
 (segment (start 35.95 24.8125) (end 36.3 24.8125) (width 1.53) (layer "F.Cu") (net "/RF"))
 (segment (start 34.585 26.8) (end 34.585 27.05) (width 1.3) (layer "F.Cu") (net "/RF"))
 (segment (start 34.585 28.65) (end 34.585 29.85) (width 0.94) (layer "F.Cu") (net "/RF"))
 (segment (start 32.05 32.3) (end 32.05 36.2) (width 0.94) (layer "F.Cu") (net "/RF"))
 (segment (start 34.585 29.85) (end 44.7 29.85) (width 0.94) (layer "F.Cu") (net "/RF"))
 (segment (start 35.1 24.8125) (end 35.55 24.8125) (width 2.17) (layer "F.Cu") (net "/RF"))
 (segment (start 34.585 27.25) (end 34.585 27.5) (width 1.26) (layer "F.Cu") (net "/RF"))
 (segment (start 37.85 24.8125) (end 38.3 24.8125) (width 1.46) (layer "F.Cu") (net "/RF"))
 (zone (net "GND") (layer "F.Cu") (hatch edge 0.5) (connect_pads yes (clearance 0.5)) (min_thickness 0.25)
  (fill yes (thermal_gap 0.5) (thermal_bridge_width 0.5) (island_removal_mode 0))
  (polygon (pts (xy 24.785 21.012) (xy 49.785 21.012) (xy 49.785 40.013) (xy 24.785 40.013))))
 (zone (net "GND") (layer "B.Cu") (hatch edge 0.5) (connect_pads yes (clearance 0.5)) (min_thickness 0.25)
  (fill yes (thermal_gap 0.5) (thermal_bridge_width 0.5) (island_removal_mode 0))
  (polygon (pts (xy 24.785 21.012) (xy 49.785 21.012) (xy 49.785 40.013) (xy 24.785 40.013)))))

